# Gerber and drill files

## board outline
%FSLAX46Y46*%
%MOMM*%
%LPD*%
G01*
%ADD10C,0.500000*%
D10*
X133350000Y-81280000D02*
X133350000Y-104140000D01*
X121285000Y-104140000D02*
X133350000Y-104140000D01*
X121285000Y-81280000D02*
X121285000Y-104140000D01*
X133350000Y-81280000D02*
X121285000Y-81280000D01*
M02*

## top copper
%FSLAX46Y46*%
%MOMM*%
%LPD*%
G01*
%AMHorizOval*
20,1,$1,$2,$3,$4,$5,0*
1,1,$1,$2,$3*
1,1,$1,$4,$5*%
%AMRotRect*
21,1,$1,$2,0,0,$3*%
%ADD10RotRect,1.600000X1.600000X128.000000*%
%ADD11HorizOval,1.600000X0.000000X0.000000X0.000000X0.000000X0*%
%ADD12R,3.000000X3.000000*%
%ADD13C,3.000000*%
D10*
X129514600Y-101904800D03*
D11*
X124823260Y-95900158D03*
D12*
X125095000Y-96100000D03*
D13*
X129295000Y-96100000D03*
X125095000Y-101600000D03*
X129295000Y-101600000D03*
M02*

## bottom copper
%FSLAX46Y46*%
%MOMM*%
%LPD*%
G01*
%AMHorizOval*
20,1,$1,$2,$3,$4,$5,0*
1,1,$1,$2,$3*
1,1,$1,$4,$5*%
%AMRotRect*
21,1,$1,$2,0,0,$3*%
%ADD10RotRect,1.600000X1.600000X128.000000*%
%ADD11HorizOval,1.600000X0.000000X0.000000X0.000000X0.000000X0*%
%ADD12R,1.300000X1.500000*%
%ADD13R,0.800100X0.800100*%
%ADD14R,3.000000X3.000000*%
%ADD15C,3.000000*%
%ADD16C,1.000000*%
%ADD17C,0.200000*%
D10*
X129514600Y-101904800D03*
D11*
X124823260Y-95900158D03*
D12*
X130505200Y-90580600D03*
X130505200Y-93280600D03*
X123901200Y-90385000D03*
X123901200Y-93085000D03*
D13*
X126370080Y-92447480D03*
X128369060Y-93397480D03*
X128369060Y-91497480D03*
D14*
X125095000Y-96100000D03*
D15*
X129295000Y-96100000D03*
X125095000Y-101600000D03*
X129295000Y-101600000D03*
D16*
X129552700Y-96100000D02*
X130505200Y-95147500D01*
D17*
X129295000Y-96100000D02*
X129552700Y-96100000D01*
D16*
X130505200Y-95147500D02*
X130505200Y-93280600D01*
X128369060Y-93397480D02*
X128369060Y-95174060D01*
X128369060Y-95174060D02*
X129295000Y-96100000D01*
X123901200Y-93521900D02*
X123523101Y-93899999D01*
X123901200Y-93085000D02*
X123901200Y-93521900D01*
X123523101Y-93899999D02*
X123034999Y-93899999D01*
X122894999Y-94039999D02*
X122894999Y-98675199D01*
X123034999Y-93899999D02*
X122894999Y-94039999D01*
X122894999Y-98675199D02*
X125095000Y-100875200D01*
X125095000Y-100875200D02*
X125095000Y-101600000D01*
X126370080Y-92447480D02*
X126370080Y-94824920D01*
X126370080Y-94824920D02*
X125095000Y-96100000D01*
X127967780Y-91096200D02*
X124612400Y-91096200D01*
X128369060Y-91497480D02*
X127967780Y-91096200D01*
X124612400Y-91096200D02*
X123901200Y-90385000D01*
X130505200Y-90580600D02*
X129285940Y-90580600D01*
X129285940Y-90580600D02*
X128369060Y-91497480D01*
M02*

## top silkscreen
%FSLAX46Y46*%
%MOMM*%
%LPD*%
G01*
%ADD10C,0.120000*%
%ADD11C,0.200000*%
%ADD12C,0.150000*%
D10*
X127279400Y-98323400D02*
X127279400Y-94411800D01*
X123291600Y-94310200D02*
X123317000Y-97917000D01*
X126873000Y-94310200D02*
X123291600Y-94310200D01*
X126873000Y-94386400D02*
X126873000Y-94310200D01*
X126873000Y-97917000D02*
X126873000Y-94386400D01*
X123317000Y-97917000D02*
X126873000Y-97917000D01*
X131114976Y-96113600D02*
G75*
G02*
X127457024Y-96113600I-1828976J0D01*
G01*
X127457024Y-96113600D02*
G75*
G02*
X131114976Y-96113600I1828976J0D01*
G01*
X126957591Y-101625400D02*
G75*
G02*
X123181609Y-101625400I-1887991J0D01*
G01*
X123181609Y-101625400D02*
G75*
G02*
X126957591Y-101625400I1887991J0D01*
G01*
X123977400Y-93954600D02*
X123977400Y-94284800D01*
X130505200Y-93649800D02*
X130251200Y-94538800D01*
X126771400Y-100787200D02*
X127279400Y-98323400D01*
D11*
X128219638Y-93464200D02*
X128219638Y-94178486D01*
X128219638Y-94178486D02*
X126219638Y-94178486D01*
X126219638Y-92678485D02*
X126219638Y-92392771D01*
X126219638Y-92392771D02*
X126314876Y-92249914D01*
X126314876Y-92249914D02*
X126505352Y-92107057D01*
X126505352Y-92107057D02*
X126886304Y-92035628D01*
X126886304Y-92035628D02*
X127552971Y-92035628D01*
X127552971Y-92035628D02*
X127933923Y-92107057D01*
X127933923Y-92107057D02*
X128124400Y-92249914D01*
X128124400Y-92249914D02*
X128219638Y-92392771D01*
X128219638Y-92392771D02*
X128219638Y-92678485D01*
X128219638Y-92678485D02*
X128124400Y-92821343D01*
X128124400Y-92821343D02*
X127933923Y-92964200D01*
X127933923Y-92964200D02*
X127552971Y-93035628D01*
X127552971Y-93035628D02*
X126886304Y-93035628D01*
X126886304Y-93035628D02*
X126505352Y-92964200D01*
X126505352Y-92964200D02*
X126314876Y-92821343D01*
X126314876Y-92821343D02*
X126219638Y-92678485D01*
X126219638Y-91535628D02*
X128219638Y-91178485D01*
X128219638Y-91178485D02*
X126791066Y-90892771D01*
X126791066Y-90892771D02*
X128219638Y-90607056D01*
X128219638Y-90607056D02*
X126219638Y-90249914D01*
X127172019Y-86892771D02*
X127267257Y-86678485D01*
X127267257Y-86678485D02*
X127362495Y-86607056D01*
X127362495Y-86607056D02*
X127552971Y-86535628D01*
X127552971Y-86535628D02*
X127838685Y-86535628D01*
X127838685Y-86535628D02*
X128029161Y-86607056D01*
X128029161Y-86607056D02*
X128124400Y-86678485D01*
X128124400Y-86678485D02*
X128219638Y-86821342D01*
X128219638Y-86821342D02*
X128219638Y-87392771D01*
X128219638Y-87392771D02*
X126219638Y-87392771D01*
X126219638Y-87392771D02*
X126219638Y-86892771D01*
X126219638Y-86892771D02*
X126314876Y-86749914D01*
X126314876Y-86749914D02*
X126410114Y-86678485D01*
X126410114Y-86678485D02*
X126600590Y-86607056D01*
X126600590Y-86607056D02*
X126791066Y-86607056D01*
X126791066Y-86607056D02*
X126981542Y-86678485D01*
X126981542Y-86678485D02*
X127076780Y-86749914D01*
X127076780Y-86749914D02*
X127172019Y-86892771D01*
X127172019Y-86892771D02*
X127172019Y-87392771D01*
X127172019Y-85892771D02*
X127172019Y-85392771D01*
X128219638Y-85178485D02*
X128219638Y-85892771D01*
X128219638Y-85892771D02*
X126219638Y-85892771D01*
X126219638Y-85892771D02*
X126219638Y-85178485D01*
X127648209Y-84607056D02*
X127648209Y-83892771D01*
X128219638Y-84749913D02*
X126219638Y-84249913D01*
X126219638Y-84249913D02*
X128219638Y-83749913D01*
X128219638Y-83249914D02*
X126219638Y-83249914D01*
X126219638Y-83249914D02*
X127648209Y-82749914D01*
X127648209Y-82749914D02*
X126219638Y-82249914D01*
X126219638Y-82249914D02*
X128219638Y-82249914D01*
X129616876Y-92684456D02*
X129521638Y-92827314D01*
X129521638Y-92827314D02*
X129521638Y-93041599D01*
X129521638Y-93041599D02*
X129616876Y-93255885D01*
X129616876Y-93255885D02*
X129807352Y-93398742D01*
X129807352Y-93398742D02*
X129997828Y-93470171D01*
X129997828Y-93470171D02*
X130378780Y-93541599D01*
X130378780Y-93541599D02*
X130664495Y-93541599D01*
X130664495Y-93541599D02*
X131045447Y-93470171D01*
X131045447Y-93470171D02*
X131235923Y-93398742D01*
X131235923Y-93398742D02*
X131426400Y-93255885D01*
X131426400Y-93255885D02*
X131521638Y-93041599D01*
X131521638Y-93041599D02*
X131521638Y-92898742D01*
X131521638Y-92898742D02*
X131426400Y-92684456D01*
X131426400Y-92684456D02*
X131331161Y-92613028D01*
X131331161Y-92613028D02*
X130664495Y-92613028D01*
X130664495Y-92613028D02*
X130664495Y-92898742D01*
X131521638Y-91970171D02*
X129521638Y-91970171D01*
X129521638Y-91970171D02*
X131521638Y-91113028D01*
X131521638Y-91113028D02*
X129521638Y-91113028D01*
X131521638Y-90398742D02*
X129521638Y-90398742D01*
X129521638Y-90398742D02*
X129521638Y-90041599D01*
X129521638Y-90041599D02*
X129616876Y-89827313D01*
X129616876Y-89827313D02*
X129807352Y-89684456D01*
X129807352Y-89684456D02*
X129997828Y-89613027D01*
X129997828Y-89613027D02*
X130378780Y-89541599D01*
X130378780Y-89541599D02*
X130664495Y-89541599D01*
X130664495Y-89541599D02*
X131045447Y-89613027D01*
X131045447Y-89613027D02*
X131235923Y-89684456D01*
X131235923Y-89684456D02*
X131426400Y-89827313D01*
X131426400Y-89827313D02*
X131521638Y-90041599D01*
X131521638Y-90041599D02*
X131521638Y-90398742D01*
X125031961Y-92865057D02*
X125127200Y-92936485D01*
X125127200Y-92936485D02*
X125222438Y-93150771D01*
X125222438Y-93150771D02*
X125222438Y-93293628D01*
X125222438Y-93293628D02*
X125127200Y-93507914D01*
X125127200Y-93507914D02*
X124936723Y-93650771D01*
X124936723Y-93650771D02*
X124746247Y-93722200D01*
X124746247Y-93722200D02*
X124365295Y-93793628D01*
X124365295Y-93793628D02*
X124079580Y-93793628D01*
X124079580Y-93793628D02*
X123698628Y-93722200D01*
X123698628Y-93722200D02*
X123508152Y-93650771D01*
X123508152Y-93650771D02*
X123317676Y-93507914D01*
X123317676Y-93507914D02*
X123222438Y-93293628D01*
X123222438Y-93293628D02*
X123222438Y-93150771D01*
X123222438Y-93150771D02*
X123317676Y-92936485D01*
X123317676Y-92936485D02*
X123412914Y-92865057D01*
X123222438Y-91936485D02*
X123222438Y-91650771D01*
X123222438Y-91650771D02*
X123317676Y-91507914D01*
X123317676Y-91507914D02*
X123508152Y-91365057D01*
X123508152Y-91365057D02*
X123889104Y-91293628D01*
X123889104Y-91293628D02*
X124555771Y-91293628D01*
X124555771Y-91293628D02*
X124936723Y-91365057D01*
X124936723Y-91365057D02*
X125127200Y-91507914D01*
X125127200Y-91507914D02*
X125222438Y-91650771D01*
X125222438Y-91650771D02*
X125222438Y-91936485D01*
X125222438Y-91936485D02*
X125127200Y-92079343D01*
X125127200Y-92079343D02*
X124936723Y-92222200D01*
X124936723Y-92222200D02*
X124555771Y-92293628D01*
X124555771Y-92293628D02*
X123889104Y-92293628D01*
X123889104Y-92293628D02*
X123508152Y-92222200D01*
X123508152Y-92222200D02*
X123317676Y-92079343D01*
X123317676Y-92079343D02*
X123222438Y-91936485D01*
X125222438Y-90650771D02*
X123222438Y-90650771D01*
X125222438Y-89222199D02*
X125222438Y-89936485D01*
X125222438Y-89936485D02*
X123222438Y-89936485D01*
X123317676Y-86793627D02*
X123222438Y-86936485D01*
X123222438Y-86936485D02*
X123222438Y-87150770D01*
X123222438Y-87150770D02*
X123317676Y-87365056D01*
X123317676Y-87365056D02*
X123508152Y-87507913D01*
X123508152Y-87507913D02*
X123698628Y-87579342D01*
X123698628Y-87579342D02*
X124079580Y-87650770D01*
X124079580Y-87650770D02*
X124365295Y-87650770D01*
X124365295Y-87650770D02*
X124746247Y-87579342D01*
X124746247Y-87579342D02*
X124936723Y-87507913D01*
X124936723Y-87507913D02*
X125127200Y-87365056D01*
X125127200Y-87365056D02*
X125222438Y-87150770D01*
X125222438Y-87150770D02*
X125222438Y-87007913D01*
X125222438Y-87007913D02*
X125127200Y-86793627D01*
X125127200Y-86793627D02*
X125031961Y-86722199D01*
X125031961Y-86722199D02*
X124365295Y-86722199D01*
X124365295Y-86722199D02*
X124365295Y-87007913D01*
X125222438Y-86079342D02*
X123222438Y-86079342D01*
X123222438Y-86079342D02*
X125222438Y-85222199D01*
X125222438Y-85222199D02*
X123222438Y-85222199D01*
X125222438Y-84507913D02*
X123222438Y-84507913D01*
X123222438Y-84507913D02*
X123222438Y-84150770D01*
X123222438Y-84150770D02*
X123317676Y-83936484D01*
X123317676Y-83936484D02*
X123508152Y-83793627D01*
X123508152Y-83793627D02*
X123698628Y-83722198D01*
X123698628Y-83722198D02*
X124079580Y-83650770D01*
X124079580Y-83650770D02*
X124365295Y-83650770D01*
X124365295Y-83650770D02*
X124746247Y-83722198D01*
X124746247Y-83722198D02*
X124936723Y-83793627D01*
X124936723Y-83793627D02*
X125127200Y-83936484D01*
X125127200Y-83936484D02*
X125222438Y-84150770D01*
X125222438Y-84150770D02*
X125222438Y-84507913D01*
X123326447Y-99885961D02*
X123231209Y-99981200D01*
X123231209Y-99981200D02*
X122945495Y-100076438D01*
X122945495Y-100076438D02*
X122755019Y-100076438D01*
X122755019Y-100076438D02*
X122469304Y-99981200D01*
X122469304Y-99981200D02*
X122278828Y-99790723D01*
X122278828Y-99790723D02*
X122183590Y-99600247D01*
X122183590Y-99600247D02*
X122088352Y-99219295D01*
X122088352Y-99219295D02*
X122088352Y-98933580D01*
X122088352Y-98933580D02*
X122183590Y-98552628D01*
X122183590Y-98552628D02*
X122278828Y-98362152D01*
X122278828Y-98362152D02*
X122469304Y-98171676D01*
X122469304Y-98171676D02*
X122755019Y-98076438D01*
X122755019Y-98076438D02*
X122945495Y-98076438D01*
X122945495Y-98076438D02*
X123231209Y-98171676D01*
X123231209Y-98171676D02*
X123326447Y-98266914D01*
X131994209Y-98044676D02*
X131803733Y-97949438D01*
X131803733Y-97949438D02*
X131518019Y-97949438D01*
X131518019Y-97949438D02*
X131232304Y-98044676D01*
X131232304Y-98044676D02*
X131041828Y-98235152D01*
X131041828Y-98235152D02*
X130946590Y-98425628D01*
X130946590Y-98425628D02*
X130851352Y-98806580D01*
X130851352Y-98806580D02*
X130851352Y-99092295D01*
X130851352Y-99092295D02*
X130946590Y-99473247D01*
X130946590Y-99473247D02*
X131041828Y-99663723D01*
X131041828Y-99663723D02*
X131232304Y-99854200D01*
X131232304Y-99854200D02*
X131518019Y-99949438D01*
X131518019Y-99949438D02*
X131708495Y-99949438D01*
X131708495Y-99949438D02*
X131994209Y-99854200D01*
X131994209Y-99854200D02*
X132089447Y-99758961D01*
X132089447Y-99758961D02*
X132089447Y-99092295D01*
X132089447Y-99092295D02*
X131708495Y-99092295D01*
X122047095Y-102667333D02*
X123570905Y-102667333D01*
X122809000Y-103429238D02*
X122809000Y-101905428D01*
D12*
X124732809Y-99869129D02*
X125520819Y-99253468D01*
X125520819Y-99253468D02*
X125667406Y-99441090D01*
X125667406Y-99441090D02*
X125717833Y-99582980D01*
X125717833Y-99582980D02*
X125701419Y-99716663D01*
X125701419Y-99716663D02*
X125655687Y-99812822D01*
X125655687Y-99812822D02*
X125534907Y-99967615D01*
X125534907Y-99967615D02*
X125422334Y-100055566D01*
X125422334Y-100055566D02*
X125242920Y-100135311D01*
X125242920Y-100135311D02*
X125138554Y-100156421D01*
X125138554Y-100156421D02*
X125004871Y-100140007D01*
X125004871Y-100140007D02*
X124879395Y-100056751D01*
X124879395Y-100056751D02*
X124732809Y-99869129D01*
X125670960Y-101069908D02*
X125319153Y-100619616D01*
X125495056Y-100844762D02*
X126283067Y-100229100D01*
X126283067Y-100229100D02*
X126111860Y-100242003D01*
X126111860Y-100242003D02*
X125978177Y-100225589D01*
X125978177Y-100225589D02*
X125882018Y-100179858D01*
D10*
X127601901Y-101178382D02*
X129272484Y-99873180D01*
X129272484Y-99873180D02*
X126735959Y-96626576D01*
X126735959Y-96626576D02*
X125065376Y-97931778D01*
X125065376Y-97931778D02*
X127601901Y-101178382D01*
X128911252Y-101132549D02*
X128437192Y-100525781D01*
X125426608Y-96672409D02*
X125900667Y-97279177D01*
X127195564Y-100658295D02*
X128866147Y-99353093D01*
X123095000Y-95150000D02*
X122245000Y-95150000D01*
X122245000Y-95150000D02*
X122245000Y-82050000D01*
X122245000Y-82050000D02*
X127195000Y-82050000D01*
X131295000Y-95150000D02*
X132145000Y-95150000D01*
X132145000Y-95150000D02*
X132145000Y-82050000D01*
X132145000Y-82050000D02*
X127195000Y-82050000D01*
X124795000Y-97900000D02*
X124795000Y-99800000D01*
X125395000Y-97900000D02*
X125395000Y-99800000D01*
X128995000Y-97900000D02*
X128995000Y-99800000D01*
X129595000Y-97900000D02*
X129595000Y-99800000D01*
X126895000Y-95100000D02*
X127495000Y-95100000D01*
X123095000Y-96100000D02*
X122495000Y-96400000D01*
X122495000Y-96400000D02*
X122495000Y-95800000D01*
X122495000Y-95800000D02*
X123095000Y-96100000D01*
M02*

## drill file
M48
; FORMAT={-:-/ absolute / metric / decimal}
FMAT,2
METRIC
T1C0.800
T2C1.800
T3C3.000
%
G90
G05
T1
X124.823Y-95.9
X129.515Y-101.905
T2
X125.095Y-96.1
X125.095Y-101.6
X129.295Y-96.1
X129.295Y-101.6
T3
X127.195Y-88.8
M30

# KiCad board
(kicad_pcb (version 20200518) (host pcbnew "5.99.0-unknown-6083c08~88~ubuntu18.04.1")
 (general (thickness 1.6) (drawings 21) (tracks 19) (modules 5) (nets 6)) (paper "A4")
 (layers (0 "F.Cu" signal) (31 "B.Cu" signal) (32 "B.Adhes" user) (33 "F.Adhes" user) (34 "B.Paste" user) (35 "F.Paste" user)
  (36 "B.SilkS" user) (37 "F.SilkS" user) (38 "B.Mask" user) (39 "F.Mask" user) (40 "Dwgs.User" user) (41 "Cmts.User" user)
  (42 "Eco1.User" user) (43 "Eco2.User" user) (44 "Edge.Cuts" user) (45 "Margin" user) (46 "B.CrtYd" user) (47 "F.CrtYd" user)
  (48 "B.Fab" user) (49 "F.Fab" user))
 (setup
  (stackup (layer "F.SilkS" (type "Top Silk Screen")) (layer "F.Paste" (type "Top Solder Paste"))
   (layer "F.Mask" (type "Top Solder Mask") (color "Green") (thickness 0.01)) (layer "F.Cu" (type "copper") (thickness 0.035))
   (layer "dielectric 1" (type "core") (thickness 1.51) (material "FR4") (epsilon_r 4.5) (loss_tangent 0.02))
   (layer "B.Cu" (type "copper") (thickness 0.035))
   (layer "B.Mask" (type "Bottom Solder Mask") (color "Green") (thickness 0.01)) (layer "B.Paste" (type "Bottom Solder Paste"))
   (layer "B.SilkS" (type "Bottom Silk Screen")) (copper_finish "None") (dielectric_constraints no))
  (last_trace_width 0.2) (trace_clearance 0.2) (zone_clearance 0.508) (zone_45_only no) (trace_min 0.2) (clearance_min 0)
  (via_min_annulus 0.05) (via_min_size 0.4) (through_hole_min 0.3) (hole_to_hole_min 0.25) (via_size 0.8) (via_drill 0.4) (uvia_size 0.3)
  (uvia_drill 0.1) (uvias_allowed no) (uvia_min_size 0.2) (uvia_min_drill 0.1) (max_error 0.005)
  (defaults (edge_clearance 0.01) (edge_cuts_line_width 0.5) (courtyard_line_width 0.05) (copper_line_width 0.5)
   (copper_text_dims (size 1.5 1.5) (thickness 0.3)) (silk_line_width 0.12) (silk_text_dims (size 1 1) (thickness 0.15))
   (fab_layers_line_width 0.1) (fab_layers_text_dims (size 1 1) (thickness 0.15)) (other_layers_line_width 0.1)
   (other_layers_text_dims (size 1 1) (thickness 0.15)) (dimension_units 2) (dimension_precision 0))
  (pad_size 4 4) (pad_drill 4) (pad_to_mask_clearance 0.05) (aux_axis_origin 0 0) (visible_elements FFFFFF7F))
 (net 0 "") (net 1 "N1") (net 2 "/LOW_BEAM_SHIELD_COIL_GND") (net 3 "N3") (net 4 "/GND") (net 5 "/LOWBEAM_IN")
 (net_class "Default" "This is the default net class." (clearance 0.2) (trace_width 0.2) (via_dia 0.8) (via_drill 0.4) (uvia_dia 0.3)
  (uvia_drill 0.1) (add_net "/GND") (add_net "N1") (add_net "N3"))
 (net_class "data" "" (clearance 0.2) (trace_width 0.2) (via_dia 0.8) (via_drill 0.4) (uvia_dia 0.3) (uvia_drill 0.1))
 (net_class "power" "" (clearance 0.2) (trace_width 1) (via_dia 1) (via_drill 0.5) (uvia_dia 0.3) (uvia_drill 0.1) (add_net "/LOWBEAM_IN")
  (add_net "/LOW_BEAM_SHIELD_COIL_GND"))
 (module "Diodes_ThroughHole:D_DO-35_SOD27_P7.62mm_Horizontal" (layer "F.Cu") (at 129.5146 101.9048 128)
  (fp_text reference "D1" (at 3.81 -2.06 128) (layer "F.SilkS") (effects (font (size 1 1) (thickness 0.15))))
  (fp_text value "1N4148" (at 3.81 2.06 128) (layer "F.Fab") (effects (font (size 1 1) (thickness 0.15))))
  (fp_line (start 1.75 -1.06) (end 1.75 1.06) (layer "F.SilkS") (width 0.12))
  (fp_line (start 1.75 1.06) (end 5.87 1.06) (layer "F.SilkS") (width 0.12))
  (fp_line (start 5.87 1.06) (end 5.87 -1.06) (layer "F.SilkS") (width 0.12))
  (fp_line (start 5.87 -1.06) (end 1.75 -1.06) (layer "F.SilkS") (width 0.12))
  (fp_line (start 0.98 0) (end 1.75 0) (layer "F.SilkS") (width 0.12))
  (fp_line (start 6.64 0) (end 5.87 0) (layer "F.SilkS") (width 0.12))
  (fp_line (start 2.41 -1.06) (end 2.41 1.06) (layer "F.SilkS") (width 0.12))
  (pad "1" thru_hole rect (at 0 0 128) (size 1.6 1.6) (drill 0.8) (layers *.Cu *.Mask) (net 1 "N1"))
  (pad "2" thru_hole oval (at 7.62 0 128) (size 1.6 1.6) (drill 0.8) (layers *.Cu *.Mask) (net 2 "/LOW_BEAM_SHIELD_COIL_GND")))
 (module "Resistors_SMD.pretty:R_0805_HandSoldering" (layer "B.Cu") (at 130.5052 91.9306 90)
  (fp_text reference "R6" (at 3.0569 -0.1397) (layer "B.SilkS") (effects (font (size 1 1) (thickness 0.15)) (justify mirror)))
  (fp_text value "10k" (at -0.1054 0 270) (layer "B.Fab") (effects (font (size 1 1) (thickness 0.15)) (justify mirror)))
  (pad "2" smd rect (at 1.35 0 90) (size 1.5 1.3) (layers "B.Cu" "B.Paste" "B.Mask") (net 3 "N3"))
  (pad "1" smd rect (at -1.35 0 90) (size 1.5 1.3) (layers "B.Cu" "B.Paste" "B.Mask") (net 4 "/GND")))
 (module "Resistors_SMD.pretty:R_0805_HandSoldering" (layer "B.Cu") (at 123.9012 91.735 90)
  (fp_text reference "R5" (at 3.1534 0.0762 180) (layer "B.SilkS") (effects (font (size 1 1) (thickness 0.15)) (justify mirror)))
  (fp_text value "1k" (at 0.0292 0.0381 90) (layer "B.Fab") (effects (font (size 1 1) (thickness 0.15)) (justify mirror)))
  (pad "2" smd rect (at 1.35 0 90) (size 1.5 1.3) (layers "B.Cu" "B.Paste" "B.Mask") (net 3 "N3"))
  (pad "1" smd rect (at -1.35 0 90) (size 1.5 1.3) (layers "B.Cu" "B.Paste" "B.Mask") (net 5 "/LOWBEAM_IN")))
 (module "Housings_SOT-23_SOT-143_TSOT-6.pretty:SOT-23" (layer "B.Cu") (at 127.3683 92.44748 -90)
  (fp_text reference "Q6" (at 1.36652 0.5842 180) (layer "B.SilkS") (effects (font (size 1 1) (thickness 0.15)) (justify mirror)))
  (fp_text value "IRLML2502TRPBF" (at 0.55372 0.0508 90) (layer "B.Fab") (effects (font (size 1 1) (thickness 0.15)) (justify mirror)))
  (pad "3" smd rect (at 0 0.99822 270) (size 0.8001 0.8001) (layers "B.Cu" "B.Paste" "B.Mask") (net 2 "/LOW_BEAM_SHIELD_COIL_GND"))
  (pad "2" smd rect (at 0.95 -1.00076 270) (size 0.8001 0.8001) (layers "B.Cu" "B.Paste" "B.Mask") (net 4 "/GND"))
  (pad "1" smd rect (at -0.95 -1.00076 270) (size 0.8001 0.8001) (layers "B.Cu" "B.Paste" "B.Mask") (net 3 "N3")))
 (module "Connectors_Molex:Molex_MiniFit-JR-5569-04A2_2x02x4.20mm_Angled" (layer "F.Cu") (at 125.095 96.1)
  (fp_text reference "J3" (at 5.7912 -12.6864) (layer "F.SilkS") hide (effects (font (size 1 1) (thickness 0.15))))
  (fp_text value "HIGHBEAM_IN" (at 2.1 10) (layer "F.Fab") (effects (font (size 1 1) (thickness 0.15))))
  (fp_line (start -2 -0.95) (end -2.85 -0.95) (layer "F.SilkS") (width 0.12))
  (fp_line (start -2.85 -0.95) (end -2.85 -14.05) (layer "F.SilkS") (width 0.12))
  (fp_line (start -2.85 -14.05) (end 2.1 -14.05) (layer "F.SilkS") (width 0.12))
  (fp_line (start 6.2 -0.95) (end 7.05 -0.95) (layer "F.SilkS") (width 0.12))
  (fp_line (start 7.05 -0.95) (end 7.05 -14.05) (layer "F.SilkS") (width 0.12))
  (fp_line (start 7.05 -14.05) (end 2.1 -14.05) (layer "F.SilkS") (width 0.12))
  (fp_line (start -0.3 1.8) (end -0.3 3.7) (layer "F.SilkS") (width 0.12))
  (fp_line (start 0.3 1.8) (end 0.3 3.7) (layer "F.SilkS") (width 0.12))
  (fp_line (start 3.9 1.8) (end 3.9 3.7) (layer "F.SilkS") (width 0.12))
  (fp_line (start 4.5 1.8) (end 4.5 3.7) (layer "F.SilkS") (width 0.12))
  (fp_line (start 1.8 -1) (end 2.4 -1) (layer "F.SilkS") (width 0.12))
  (fp_line (start -2 0) (end -2.6 0.3) (layer "F.SilkS") (width 0.12))
  (fp_line (start -2.6 0.3) (end -2.6 -0.3) (layer "F.SilkS") (width 0.12))
  (fp_line (start -2.6 -0.3) (end -2 0) (layer "F.SilkS") (width 0.12))
  (pad "1" thru_hole rect (at 0 0) (size 3 3) (drill 1.8) (layers *.Cu *.Mask) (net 2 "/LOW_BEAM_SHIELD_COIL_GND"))
  (pad "2" thru_hole circle (at 4.2 0) (size 3 3) (drill 1.8) (layers *.Cu *.Mask) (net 4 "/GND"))
  (pad "3" thru_hole circle (at 0 5.5) (size 3 3) (drill 1.8) (layers *.Cu *.Mask) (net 5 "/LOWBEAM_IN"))
  (pad "4" thru_hole circle (at 4.2 5.5) (size 3 3) (drill 1.8) (layers *.Cu *.Mask) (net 1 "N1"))
  (pad "" np_thru_hole circle (at 2.1 -7.3) (size 3 3) (drill 3) (layers *.Cu *.Mask)))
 (gr_line (start 127.2794 98.3234) (end 127.2794 94.4118) (layer "F.SilkS") (width 0.12))
 (gr_line (start 123.2916 94.3102) (end 123.317 97.917) (layer "F.SilkS") (width 0.12))
 (gr_line (start 126.873 94.3102) (end 123.2916 94.3102) (layer "F.SilkS") (width 0.12))
 (gr_line (start 126.873 94.3864) (end 126.873 94.3102) (layer "F.SilkS") (width 0.12))
 (gr_line (start 126.873 97.917) (end 126.873 94.3864) (layer "F.SilkS") (width 0.12))
 (gr_line (start 123.317 97.917) (end 126.873 97.917) (layer "F.SilkS") (width 0.12))
 (gr_circle (center 129.286 96.1136) (end 130.7338 94.996) (layer "F.SilkS") (width 0.12))
 (gr_circle (center 125.0696 101.6254) (end 126.873 102.1842) (layer "F.SilkS") (width 0.12))
 (gr_line (start 123.9774 93.9546) (end 123.9774 94.2848) (layer "F.SilkS") (width 0.12))
 (gr_line (start 130.5052 93.6498) (end 130.2512 94.5388) (layer "F.SilkS") (width 0.12))
 (gr_line (start 126.7714 100.7872) (end 127.2794 98.3234) (layer "F.SilkS") (width 0.12))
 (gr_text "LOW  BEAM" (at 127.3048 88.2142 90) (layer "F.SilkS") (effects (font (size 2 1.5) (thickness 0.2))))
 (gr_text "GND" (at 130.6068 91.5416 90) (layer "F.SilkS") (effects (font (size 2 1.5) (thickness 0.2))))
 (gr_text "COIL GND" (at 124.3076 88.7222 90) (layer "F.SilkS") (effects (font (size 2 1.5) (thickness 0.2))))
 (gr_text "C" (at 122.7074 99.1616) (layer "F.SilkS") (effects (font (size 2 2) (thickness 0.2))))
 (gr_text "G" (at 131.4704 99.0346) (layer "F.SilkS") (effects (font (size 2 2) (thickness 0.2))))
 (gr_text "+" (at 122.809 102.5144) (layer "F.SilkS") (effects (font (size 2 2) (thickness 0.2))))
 (gr_line (start 133.35 81.28) (end 133.35 104.14) (layer "Edge.Cuts") (width 0.5))
 (gr_line (start 121.285 104.14) (end 133.35 104.14) (layer "Edge.Cuts") (width 0.5))
 (gr_line (start 121.285 81.28) (end 121.285 104.14) (layer "Edge.Cuts") (width 0.5))
 (gr_line (start 133.35 81.28) (end 121.285 81.28) (layer "Edge.Cuts") (width 0.5))
 (segment (start 129.5527 96.1) (end 130.5052 95.1475) (width 1) (layer "B.Cu") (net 4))
 (segment (start 129.295 96.1) (end 129.5527 96.1) (width 0.2) (layer "B.Cu") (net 4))
 (segment (start 130.5052 95.1475) (end 130.5052 93.2806) (width 1) (layer "B.Cu") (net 4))
 (segment (start 128.36906 93.39748) (end 128.36906 95.17406) (width 1) (layer "B.Cu") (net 4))
 (segment (start 128.36906 95.17406) (end 129.295 96.1) (width 1) (layer "B.Cu") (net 4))
 (segment (start 123.9012 93.5219) (end 123.523101 93.899999) (width 1) (layer "B.Cu") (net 5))
 (segment (start 123.9012 93.085) (end 123.9012 93.5219) (width 1) (layer "B.Cu") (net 5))
 (segment (start 123.523101 93.899999) (end 123.034999 93.899999) (width 1) (layer "B.Cu") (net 5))
 (segment (start 122.894999 94.039999) (end 122.894999 98.675199) (width 1) (layer "B.Cu") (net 5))
 (segment (start 123.034999 93.899999) (end 122.894999 94.039999) (width 1) (layer "B.Cu") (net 5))
 (segment (start 122.894999 98.675199) (end 125.095 100.8752) (width 1) (layer "B.Cu") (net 5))
 (segment (start 125.095 100.8752) (end 125.095 101.6) (width 1) (layer "B.Cu") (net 5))
 (segment (start 126.37008 92.44748) (end 126.37008 94.82492) (width 1) (layer "B.Cu") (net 2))
 (segment (start 126.37008 94.82492) (end 125.095 96.1) (width 1) (layer "B.Cu") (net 2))
 (segment (start 127.96778 91.0962) (end 124.6124 91.0962) (width 1) (layer "B.Cu") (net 3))
 (segment (start 128.36906 91.49748) (end 127.96778 91.0962) (width 1) (layer "B.Cu") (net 3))
 (segment (start 124.6124 91.0962) (end 123.9012 90.385) (width 1) (layer "B.Cu") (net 3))
 (segment (start 130.5052 90.5806) (end 129.28594 90.5806) (width 1) (layer "B.Cu") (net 3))
 (segment (start 129.28594 90.5806) (end 128.36906 91.49748) (width 1) (layer "B.Cu") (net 3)))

